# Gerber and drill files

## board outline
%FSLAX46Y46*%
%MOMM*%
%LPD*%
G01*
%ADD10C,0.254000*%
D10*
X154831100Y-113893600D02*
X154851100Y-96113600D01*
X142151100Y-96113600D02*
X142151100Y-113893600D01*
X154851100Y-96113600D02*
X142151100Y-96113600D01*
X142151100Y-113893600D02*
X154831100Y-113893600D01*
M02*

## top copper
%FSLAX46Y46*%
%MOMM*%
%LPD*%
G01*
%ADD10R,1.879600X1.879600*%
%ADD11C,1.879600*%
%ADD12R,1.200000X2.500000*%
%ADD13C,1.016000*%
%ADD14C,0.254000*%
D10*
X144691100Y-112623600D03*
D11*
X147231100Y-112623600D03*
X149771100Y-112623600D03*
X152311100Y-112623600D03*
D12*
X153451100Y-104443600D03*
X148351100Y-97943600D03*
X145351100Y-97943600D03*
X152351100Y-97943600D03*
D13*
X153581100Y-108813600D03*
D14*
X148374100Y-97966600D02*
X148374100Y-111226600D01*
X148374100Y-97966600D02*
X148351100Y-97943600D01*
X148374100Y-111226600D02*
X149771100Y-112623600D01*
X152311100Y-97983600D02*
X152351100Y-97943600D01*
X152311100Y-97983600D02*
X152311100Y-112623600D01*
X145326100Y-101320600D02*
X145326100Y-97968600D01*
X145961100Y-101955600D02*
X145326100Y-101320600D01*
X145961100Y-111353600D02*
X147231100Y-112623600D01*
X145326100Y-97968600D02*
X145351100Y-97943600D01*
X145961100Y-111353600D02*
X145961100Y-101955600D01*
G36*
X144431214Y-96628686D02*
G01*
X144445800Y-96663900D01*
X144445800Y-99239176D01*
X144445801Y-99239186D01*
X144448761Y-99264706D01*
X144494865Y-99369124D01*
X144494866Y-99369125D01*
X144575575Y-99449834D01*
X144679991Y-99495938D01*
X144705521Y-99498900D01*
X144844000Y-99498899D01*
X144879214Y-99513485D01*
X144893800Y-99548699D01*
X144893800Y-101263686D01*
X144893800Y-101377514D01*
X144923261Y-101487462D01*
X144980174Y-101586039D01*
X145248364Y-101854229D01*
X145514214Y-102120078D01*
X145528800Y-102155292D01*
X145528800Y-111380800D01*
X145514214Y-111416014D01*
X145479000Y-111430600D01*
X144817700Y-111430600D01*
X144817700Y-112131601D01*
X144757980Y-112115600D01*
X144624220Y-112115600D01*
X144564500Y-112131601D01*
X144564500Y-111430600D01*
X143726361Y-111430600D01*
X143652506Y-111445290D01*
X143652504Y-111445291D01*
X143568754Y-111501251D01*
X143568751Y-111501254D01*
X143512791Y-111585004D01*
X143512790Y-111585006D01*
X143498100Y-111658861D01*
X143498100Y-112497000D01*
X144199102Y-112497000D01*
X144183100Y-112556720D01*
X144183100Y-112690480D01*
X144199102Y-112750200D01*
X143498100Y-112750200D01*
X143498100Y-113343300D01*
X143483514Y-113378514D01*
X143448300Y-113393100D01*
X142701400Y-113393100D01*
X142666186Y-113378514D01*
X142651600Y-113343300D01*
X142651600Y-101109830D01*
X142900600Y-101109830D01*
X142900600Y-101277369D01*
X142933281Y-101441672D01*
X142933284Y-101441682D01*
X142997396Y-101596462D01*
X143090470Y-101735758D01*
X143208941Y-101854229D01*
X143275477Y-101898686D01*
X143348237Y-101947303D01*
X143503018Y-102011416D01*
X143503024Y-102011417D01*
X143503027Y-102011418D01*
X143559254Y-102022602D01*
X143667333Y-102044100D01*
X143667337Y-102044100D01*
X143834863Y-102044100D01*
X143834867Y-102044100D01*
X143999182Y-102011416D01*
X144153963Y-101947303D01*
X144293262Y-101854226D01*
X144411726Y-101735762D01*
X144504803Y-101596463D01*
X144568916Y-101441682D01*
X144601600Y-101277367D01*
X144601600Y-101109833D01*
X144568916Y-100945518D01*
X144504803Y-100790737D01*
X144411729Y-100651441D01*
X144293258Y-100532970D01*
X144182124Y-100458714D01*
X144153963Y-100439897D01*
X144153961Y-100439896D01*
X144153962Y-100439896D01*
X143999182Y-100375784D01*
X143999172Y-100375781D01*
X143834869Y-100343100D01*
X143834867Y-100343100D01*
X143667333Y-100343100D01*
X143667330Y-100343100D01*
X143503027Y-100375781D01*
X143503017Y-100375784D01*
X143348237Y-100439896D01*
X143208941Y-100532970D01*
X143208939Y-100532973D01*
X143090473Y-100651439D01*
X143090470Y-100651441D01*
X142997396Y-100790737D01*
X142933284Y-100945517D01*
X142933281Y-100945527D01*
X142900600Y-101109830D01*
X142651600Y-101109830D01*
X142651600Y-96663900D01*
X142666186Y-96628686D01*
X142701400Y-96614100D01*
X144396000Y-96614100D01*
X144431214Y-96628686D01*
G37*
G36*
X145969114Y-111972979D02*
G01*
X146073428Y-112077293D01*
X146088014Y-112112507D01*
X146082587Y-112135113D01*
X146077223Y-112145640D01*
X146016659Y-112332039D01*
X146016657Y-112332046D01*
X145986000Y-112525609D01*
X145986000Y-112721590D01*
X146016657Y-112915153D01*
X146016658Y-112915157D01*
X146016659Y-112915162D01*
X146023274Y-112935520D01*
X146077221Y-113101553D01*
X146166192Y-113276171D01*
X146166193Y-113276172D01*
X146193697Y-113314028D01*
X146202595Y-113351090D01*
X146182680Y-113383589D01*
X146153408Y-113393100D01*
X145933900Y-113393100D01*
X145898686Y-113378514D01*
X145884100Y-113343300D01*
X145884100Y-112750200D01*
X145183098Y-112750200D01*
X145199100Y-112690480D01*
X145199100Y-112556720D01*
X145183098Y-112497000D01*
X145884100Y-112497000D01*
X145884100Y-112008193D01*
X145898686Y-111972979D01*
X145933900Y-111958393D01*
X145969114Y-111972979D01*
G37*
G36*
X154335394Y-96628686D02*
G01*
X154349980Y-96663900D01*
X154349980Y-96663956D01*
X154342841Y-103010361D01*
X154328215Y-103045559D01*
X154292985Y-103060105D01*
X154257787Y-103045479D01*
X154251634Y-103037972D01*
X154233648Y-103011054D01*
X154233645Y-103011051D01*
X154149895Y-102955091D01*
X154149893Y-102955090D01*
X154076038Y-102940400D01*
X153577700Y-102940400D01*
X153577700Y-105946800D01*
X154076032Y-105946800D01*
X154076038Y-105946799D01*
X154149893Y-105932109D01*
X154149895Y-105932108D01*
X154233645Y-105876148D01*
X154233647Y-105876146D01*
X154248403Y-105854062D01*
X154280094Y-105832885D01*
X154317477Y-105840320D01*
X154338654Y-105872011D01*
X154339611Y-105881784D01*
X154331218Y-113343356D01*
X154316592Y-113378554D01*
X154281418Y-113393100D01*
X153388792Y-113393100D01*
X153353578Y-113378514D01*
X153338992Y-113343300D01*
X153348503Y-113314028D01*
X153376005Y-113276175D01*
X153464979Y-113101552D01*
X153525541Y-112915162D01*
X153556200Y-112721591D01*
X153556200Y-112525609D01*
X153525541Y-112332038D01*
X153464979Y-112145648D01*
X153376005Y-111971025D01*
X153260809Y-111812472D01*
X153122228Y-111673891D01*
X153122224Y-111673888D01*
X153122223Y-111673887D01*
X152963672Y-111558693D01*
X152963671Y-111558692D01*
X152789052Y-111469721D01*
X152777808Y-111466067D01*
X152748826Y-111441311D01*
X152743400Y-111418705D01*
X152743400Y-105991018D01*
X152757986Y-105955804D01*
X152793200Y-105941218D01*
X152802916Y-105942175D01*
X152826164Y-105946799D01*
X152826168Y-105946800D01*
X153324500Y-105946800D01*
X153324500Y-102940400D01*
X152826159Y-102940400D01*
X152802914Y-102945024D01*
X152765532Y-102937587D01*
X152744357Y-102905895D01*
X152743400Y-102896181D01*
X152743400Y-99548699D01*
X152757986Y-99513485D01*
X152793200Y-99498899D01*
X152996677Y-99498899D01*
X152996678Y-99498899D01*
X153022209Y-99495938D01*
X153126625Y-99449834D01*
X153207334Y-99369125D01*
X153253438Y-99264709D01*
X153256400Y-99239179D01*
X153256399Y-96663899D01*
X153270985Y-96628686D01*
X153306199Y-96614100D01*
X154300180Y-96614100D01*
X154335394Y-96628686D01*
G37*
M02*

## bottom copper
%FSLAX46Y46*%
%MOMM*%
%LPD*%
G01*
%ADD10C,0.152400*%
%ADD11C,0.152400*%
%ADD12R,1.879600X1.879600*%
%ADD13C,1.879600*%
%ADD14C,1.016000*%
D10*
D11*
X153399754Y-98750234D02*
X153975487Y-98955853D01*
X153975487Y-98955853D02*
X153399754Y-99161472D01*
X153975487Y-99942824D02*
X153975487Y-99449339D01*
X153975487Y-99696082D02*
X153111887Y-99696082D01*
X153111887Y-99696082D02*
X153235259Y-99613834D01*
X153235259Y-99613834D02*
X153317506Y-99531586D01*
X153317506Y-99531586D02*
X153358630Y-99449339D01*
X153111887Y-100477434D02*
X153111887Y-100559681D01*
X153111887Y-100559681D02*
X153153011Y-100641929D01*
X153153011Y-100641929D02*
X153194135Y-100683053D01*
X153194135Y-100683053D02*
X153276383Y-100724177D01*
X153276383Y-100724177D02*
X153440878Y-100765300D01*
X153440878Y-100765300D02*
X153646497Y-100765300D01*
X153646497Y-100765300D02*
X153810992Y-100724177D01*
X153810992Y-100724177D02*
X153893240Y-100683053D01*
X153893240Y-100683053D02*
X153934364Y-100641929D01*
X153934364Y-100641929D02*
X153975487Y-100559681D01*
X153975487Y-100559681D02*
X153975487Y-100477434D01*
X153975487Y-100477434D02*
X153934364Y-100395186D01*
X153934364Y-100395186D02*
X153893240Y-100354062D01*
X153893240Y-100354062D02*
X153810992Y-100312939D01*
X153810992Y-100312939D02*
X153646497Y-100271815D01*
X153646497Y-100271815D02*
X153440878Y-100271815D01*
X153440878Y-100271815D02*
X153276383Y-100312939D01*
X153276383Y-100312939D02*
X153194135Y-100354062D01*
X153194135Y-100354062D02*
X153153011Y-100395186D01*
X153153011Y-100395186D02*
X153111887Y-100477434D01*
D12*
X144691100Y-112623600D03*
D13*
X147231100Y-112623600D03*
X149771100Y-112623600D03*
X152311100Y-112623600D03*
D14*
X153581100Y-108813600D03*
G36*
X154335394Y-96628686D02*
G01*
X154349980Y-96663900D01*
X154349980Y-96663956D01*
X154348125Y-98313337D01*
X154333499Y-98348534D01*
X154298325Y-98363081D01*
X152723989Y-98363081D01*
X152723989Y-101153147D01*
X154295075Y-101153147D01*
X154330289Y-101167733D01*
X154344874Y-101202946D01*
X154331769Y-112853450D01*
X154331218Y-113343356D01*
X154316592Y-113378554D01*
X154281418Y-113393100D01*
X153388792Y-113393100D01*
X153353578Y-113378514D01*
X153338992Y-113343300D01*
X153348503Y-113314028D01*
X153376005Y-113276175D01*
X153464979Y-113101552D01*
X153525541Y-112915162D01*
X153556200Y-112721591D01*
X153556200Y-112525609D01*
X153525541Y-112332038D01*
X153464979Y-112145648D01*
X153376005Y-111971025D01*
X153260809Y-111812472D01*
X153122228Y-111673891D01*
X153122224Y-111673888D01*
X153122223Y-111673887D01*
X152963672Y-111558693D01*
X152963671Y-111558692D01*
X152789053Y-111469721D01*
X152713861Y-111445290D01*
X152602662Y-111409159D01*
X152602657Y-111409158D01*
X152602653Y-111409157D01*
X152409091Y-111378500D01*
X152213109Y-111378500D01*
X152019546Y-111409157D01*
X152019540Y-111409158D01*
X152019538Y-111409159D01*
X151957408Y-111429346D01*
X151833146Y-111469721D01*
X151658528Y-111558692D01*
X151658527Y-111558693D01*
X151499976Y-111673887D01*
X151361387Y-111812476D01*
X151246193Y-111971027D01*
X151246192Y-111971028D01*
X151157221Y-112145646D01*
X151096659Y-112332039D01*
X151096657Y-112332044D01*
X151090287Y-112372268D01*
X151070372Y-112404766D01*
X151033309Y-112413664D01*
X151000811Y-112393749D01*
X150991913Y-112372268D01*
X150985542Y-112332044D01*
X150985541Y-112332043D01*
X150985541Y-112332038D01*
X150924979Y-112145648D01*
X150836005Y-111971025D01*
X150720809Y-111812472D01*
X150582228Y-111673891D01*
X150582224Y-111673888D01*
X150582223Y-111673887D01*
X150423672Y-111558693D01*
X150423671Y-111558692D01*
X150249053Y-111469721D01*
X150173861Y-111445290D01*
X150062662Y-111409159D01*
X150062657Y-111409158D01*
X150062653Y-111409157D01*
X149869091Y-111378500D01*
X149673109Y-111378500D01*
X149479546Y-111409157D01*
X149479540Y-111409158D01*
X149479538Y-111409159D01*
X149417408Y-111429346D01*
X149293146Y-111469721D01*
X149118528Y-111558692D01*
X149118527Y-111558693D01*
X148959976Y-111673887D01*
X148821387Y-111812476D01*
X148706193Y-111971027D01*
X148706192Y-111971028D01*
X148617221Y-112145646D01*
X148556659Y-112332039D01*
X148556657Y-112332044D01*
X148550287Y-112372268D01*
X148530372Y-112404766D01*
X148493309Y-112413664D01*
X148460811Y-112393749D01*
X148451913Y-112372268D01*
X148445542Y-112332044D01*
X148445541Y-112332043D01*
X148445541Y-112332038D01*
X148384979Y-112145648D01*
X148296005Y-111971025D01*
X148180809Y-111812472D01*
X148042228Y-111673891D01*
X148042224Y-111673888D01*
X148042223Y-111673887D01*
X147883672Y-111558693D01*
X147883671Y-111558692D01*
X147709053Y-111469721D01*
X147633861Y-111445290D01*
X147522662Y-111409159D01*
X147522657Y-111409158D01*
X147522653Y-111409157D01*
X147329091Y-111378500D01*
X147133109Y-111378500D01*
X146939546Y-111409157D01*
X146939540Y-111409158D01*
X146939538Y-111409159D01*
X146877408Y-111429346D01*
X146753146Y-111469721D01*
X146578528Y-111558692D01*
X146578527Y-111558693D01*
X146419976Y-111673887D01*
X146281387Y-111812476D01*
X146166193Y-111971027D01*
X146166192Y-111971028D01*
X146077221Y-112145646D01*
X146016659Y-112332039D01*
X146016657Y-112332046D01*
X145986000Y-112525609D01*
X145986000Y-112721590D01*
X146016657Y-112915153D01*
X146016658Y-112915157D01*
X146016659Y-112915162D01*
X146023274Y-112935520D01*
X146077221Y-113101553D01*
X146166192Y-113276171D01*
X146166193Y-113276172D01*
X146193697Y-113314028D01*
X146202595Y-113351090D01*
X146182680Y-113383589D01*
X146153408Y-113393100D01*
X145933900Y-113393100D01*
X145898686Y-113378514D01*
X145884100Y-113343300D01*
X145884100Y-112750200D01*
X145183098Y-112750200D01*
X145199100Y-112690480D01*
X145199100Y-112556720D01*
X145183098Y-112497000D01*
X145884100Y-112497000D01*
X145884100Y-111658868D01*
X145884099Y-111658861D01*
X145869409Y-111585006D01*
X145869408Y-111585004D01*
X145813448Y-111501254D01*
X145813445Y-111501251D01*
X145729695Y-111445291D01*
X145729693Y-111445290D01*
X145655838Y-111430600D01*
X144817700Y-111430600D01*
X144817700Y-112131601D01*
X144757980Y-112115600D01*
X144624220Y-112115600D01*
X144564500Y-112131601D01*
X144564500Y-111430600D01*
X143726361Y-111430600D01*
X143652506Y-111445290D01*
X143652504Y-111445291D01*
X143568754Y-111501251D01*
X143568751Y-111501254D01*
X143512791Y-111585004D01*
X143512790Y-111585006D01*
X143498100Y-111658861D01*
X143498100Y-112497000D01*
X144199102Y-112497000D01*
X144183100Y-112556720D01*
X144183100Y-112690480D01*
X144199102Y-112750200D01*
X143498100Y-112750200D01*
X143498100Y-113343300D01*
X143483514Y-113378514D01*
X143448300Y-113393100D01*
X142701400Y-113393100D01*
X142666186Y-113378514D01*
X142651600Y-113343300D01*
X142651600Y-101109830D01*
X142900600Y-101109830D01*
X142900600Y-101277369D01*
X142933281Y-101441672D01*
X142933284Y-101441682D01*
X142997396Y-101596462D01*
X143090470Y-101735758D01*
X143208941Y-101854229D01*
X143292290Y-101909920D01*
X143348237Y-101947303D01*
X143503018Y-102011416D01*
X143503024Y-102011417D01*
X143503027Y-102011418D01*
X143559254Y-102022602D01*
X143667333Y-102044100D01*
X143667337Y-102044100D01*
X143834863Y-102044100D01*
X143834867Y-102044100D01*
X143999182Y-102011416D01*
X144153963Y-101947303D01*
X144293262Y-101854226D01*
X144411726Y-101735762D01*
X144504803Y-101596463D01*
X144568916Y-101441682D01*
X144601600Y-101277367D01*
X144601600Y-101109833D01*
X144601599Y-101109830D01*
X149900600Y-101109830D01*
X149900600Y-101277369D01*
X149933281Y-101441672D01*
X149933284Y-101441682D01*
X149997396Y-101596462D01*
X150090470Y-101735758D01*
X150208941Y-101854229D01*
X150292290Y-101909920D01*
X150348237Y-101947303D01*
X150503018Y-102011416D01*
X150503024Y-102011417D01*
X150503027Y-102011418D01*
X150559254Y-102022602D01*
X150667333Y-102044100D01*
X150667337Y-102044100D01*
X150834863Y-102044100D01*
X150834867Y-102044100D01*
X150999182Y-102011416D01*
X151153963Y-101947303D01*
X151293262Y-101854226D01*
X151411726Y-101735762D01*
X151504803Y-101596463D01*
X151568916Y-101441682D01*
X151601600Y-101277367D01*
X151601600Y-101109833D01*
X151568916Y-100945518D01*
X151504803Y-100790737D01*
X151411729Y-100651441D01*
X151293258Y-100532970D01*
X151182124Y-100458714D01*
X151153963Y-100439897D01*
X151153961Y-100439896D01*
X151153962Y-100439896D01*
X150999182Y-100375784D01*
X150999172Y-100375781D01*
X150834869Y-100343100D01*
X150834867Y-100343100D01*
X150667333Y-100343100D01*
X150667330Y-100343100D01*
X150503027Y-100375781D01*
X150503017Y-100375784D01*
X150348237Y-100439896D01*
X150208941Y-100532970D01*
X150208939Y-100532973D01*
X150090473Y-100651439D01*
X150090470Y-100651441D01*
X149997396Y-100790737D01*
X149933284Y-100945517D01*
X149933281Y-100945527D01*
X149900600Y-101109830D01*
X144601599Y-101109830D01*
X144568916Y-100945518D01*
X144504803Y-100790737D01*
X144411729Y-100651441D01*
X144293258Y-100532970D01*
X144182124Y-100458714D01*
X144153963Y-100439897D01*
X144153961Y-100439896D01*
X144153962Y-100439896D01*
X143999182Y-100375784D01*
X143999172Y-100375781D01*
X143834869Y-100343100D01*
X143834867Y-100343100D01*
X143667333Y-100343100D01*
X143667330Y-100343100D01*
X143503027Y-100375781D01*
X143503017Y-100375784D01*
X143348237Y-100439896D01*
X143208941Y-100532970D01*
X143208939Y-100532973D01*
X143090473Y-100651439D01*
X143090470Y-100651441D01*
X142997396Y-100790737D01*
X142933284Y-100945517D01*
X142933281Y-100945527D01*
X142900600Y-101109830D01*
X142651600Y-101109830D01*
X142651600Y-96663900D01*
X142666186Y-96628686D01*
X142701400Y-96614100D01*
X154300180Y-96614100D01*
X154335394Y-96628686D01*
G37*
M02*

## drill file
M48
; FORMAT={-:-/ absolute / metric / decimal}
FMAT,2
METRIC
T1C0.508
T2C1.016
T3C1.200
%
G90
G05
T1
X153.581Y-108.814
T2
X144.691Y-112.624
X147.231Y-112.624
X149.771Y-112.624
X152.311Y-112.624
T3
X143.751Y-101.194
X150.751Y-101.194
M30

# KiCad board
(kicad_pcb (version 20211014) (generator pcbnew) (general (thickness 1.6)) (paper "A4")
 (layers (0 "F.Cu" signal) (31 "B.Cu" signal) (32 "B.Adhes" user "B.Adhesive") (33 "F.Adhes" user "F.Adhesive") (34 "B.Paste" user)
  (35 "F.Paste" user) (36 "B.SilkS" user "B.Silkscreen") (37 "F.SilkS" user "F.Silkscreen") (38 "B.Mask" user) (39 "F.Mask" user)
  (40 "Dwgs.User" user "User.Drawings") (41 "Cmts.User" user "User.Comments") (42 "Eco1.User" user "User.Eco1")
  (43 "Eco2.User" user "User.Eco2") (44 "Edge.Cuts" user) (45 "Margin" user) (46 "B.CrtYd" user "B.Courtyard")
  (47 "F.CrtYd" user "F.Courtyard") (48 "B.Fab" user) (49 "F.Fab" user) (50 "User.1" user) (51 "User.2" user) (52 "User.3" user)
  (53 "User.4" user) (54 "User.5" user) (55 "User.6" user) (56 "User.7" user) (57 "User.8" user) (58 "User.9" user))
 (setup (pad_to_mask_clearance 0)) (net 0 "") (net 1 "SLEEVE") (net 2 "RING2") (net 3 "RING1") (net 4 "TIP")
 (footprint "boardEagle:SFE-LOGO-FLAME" (layer "F.Cu") (at 153.8351 107.6706 90)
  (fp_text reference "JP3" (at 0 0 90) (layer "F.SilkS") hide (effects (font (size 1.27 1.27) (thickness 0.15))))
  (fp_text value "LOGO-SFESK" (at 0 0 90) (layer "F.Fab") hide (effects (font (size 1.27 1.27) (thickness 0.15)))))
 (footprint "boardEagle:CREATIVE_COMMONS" (layer "F.Cu") (at 138.3411 125.3236)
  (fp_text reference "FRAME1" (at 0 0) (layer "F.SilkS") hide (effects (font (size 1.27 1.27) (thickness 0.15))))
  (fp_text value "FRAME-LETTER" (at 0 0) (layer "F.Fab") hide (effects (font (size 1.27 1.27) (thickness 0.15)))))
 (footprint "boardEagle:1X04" (layer "F.Cu") (at 144.6911 112.6236)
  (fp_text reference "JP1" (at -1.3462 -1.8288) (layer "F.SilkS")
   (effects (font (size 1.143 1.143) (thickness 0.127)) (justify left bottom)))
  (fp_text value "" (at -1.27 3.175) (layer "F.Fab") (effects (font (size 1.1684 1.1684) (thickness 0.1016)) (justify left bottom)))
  (pad "1" thru_hole rect (at 0 0 90) (size 1.8796 1.8796) (drill 1.016) (layers *.Cu *.Mask) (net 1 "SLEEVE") (solder_mask_margin 0.1016))
  (pad "2" thru_hole circle (at 2.54 0 90) (size 1.8796 1.8796) (drill 1.016) (layers *.Cu *.Mask) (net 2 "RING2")
   (solder_mask_margin 0.1016))
  (pad "3" thru_hole circle (at 5.08 0 90) (size 1.8796 1.8796) (drill 1.016) (layers *.Cu *.Mask) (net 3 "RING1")
   (solder_mask_margin 0.1016))
  (pad "4" thru_hole circle (at 7.62 0 90) (size 1.8796 1.8796) (drill 1.016) (layers *.Cu *.Mask) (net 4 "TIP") (solder_mask_margin 0.1016)))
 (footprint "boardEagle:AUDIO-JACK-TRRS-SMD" (layer "F.Cu") (at 142.1511 101.1936)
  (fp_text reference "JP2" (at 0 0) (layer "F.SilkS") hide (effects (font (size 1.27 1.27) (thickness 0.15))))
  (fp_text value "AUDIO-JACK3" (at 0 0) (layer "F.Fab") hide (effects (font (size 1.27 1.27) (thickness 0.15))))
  (pad "" np_thru_hole circle (at 1.6 0) (size 1.2 1.2) (drill 1.2) (layers *.Cu *.Mask))
  (pad "" np_thru_hole circle (at 8.6 0) (size 1.2 1.2) (drill 1.2) (layers *.Cu *.Mask))
  (pad "EARTH" smd rect (at 11.3 3.25) (size 1.2 2.5) (layers "F.Cu" "F.Paste" "F.Mask") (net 1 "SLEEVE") (solder_mask_margin 0.1016))
  (pad "RING1" smd rect (at 6.2 -3.25) (size 1.2 2.5) (layers "F.Cu" "F.Paste" "F.Mask") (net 3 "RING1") (solder_mask_margin 0.1016))
  (pad "RING2" smd rect (at 3.2 -3.25 180) (size 1.2 2.5) (layers "F.Cu" "F.Paste" "F.Mask") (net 2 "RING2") (solder_mask_margin 0.1016))
  (pad "TIP" smd rect (at 10.2 -3.25) (size 1.2 2.5) (layers "F.Cu" "F.Paste" "F.Mask") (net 4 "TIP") (solder_mask_margin 0.1016)))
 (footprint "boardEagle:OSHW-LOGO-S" (layer "B.Cu") (at 151.0411 103.9876 -90)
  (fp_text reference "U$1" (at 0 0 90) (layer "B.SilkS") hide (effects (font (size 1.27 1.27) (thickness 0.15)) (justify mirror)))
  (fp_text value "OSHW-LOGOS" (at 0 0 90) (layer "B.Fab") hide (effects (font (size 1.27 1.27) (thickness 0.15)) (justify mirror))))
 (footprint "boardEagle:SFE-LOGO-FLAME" (layer "B.Cu") (at 152.3111 106.2736 -90)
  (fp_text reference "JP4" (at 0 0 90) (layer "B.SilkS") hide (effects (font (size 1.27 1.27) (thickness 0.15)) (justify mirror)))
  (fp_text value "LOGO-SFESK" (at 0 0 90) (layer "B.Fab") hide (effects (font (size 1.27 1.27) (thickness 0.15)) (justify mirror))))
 (gr_line (start 154.8311 113.8936) (end 154.8511 96.1136) (layer "Edge.Cuts") (width 0.254))
 (gr_line (start 142.1511 96.1136) (end 142.1511 113.8936) (layer "Edge.Cuts") (width 0.254))
 (gr_line (start 154.8511 96.1136) (end 142.1511 96.1136) (layer "Edge.Cuts") (width 0.254))
 (gr_line (start 142.1511 113.8936) (end 154.8311 113.8936) (layer "Edge.Cuts") (width 0.254))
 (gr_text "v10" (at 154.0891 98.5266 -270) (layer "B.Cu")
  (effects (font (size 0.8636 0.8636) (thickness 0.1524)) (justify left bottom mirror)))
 (segment (start 148.3741 97.9666) (end 148.3741 111.2266) (width 0.254) (layer "F.Cu") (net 3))
 (segment (start 148.3741 97.9666) (end 148.3511 97.9436) (width 0.254) (layer "F.Cu") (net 3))
 (segment (start 148.3741 111.2266) (end 149.7711 112.6236) (width 0.254) (layer "F.Cu") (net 3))
 (segment (start 152.3111 97.9836) (end 152.3511 97.9436) (width 0.254) (layer "F.Cu") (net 4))
 (segment (start 152.3111 97.9836) (end 152.3111 112.6236) (width 0.254) (layer "F.Cu") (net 4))
 (segment (start 145.3261 101.3206) (end 145.3261 97.9686) (width 0.254) (layer "F.Cu") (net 2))
 (segment (start 145.9611 101.9556) (end 145.3261 101.3206) (width 0.254) (layer "F.Cu") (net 2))
 (segment (start 145.9611 111.3536) (end 147.2311 112.6236) (width 0.254) (layer "F.Cu") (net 2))
 (segment (start 145.3261 97.9686) (end 145.3511 97.9436) (width 0.254) (layer "F.Cu") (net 2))
 (segment (start 145.9611 111.3536) (end 145.9611 101.9556) (width 0.254) (layer "F.Cu") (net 2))
 (via (at 153.5811 108.8136) (size 1.016) (drill 0.508) (layers "F.Cu" "B.Cu") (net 1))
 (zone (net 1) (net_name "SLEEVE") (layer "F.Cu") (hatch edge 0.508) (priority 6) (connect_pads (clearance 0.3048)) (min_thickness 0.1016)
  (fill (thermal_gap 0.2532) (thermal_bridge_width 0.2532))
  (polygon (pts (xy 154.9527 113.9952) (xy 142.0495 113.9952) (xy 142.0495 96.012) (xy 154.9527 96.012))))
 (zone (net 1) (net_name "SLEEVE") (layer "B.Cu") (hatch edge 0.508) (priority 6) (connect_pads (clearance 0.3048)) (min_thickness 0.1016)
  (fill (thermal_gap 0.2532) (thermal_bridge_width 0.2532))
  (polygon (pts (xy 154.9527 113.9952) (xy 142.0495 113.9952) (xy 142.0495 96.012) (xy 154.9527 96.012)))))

